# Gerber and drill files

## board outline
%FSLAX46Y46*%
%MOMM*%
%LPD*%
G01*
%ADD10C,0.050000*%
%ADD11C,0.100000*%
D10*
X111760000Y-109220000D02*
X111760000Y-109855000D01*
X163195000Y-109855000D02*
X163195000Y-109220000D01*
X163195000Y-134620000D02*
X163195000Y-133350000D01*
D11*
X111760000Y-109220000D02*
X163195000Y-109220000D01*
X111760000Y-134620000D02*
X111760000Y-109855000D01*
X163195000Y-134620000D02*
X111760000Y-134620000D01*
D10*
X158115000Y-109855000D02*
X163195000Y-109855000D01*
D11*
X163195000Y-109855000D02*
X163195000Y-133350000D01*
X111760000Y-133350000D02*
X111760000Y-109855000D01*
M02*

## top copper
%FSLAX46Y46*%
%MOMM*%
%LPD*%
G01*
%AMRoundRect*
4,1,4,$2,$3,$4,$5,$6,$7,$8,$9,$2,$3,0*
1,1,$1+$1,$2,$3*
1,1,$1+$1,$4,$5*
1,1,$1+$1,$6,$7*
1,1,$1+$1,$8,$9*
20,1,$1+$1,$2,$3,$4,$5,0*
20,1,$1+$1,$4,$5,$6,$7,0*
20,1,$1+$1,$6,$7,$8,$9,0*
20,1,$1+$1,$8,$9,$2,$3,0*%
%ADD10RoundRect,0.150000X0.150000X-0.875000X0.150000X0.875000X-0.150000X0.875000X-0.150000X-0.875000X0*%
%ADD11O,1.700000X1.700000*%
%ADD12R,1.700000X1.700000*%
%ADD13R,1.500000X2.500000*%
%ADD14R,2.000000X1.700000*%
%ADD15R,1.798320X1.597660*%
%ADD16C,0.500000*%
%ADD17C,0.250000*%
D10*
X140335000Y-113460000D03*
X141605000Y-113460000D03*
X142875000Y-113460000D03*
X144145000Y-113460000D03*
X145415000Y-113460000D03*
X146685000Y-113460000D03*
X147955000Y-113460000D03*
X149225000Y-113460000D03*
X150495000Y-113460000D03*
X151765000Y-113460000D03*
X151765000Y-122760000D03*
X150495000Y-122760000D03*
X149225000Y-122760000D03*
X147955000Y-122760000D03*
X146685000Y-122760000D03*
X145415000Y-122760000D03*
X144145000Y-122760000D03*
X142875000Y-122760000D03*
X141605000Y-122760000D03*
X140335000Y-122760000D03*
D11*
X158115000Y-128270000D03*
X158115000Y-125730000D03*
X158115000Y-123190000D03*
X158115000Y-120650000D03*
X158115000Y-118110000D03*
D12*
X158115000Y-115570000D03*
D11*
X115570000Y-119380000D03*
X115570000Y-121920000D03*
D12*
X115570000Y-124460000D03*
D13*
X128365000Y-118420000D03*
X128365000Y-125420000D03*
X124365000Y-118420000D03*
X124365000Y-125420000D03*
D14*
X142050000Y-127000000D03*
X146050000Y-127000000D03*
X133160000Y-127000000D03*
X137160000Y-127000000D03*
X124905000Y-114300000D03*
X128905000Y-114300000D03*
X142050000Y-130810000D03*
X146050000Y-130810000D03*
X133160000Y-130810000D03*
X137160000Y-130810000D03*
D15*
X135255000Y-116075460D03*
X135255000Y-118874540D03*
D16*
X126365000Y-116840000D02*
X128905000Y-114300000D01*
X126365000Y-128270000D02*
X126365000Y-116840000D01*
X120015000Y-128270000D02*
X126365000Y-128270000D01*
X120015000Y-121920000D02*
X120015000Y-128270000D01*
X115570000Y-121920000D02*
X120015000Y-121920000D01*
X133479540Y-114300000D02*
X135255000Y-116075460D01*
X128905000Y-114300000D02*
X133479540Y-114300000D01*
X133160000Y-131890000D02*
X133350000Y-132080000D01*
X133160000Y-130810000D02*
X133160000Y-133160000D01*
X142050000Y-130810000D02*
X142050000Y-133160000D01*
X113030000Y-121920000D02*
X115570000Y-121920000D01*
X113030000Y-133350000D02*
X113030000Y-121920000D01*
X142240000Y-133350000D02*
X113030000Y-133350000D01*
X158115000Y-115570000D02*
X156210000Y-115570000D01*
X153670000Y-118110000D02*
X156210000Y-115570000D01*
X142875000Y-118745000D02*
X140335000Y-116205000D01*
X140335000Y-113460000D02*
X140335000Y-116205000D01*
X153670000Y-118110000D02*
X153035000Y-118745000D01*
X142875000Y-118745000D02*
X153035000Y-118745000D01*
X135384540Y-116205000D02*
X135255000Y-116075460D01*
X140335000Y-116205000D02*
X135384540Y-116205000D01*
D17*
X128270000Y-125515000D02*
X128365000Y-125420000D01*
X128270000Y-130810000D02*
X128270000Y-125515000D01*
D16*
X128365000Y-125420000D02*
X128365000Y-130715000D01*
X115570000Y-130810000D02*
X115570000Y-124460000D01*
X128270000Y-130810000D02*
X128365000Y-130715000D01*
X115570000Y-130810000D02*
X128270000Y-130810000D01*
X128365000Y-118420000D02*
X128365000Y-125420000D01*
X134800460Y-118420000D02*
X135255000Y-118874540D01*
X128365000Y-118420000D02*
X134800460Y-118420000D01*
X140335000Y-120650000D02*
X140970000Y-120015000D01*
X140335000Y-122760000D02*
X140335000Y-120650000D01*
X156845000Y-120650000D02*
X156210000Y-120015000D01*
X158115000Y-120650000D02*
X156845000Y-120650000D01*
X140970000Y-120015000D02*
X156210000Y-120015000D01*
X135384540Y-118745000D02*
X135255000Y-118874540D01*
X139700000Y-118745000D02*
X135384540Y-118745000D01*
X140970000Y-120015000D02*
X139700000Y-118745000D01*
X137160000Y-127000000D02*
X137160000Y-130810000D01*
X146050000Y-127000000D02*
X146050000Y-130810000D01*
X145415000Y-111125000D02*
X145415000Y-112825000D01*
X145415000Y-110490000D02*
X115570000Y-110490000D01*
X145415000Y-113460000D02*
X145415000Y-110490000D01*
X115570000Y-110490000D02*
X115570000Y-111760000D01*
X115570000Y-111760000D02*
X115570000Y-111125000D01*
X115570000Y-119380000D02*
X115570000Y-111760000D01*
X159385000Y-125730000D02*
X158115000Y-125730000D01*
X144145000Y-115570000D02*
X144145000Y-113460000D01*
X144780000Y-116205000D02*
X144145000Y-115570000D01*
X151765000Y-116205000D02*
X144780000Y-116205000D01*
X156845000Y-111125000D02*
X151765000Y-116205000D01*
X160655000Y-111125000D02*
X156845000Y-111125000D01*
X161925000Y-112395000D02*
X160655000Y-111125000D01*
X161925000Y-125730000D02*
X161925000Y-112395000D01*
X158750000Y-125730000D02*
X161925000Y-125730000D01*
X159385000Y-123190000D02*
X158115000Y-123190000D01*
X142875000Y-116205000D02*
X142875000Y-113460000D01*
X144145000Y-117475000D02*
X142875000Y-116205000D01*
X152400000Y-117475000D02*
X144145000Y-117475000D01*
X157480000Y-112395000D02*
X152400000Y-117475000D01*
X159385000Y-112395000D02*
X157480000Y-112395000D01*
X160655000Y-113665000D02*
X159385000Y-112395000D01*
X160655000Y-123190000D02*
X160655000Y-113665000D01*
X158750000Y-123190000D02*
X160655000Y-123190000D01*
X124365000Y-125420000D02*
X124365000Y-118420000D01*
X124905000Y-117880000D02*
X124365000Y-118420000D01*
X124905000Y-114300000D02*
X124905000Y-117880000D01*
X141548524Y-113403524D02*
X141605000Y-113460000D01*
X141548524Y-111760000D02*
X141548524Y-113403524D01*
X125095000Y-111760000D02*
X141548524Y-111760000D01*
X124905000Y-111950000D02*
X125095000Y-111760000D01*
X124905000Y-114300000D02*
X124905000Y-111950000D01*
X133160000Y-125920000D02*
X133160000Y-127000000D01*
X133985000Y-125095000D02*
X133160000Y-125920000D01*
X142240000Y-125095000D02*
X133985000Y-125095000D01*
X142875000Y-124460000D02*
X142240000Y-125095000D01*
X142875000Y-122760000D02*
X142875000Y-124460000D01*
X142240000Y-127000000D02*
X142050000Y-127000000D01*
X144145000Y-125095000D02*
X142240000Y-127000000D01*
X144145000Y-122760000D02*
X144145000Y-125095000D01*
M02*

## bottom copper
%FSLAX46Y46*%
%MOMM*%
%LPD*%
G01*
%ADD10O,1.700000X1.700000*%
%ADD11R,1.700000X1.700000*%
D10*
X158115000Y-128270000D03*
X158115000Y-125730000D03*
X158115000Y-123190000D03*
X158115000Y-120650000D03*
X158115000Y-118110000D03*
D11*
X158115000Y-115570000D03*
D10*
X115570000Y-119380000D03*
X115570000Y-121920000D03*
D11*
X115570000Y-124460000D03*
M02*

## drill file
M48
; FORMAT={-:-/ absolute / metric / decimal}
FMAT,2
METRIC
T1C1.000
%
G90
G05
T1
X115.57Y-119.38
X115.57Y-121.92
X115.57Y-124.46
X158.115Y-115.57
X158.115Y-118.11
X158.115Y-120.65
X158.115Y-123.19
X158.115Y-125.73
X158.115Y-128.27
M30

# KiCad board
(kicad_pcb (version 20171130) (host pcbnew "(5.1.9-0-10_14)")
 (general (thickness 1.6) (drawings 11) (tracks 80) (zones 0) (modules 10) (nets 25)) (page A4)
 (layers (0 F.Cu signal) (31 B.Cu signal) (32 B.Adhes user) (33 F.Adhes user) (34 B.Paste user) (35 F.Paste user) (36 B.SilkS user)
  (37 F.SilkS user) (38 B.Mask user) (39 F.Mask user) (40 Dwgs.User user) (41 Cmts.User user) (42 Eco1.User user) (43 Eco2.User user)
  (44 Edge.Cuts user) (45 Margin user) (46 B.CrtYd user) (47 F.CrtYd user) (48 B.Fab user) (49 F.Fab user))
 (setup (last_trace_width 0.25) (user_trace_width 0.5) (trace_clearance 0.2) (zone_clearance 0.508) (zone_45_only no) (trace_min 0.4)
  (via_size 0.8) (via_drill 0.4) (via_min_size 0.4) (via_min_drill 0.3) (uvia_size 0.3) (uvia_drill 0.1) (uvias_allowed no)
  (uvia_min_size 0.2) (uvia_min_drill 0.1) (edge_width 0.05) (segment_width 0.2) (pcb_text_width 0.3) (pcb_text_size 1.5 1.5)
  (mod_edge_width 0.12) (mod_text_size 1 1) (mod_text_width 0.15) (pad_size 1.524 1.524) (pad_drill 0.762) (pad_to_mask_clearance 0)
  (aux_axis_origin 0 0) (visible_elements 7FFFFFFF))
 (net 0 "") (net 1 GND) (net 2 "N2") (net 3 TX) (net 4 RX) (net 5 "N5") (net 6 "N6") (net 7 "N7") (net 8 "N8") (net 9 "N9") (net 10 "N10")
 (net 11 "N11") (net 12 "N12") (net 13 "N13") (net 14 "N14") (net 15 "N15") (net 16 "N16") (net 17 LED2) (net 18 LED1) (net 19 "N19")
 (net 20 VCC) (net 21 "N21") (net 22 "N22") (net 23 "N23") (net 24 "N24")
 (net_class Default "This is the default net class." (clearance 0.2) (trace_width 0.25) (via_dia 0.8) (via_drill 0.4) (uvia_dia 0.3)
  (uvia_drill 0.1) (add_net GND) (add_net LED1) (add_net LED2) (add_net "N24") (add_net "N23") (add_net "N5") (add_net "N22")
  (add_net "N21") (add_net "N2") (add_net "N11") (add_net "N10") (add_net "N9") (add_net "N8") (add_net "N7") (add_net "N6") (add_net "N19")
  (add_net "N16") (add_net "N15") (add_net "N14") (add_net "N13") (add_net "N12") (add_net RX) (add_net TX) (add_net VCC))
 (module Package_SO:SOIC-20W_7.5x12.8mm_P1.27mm (layer F.Cu) (at 146.05 118.11 90)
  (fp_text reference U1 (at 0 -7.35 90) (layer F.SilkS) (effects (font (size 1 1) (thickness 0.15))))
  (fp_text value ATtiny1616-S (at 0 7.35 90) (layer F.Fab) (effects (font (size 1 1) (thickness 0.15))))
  (pad 20 smd roundrect (at 4.65 -5.715 90) (size 2.05 0.6) (layers F.Cu F.Paste F.Mask) (roundrect_rratio 0.25) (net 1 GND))
  (pad 19 smd roundrect (at 4.65 -4.445 90) (size 2.05 0.6) (layers F.Cu F.Paste F.Mask) (roundrect_rratio 0.25) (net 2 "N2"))
  (pad 18 smd roundrect (at 4.65 -3.175 90) (size 2.05 0.6) (layers F.Cu F.Paste F.Mask) (roundrect_rratio 0.25) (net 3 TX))
  (pad 17 smd roundrect (at 4.65 -1.905 90) (size 2.05 0.6) (layers F.Cu F.Paste F.Mask) (roundrect_rratio 0.25) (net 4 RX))
  (pad 16 smd roundrect (at 4.65 -0.635 90) (size 2.05 0.6) (layers F.Cu F.Paste F.Mask) (roundrect_rratio 0.25) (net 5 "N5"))
  (pad 15 smd roundrect (at 4.65 0.635 90) (size 2.05 0.6) (layers F.Cu F.Paste F.Mask) (roundrect_rratio 0.25) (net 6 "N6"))
  (pad 14 smd roundrect (at 4.65 1.905 90) (size 2.05 0.6) (layers F.Cu F.Paste F.Mask) (roundrect_rratio 0.25) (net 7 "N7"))
  (pad 13 smd roundrect (at 4.65 3.175 90) (size 2.05 0.6) (layers F.Cu F.Paste F.Mask) (roundrect_rratio 0.25) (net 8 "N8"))
  (pad 12 smd roundrect (at 4.65 4.445 90) (size 2.05 0.6) (layers F.Cu F.Paste F.Mask) (roundrect_rratio 0.25) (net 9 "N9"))
  (pad 11 smd roundrect (at 4.65 5.715 90) (size 2.05 0.6) (layers F.Cu F.Paste F.Mask) (roundrect_rratio 0.25) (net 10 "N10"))
  (pad 10 smd roundrect (at -4.65 5.715 90) (size 2.05 0.6) (layers F.Cu F.Paste F.Mask) (roundrect_rratio 0.25) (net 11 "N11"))
  (pad 9 smd roundrect (at -4.65 4.445 90) (size 2.05 0.6) (layers F.Cu F.Paste F.Mask) (roundrect_rratio 0.25) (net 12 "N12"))
  (pad 8 smd roundrect (at -4.65 3.175 90) (size 2.05 0.6) (layers F.Cu F.Paste F.Mask) (roundrect_rratio 0.25) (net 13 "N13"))
  (pad 7 smd roundrect (at -4.65 1.905 90) (size 2.05 0.6) (layers F.Cu F.Paste F.Mask) (roundrect_rratio 0.25) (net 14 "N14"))
  (pad 6 smd roundrect (at -4.65 0.635 90) (size 2.05 0.6) (layers F.Cu F.Paste F.Mask) (roundrect_rratio 0.25) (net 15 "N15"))
  (pad 5 smd roundrect (at -4.65 -0.635 90) (size 2.05 0.6) (layers F.Cu F.Paste F.Mask) (roundrect_rratio 0.25) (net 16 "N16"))
  (pad 4 smd roundrect (at -4.65 -1.905 90) (size 2.05 0.6) (layers F.Cu F.Paste F.Mask) (roundrect_rratio 0.25) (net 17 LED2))
  (pad 3 smd roundrect (at -4.65 -3.175 90) (size 2.05 0.6) (layers F.Cu F.Paste F.Mask) (roundrect_rratio 0.25) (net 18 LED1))
  (pad 2 smd roundrect (at -4.65 -4.445 90) (size 2.05 0.6) (layers F.Cu F.Paste F.Mask) (roundrect_rratio 0.25) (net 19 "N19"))
  (pad 1 smd roundrect (at -4.65 -5.715 90) (size 2.05 0.6) (layers F.Cu F.Paste F.Mask) (roundrect_rratio 0.25) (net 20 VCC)))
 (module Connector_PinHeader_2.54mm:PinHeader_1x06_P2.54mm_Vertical (layer F.Cu) (at 158.115 115.57)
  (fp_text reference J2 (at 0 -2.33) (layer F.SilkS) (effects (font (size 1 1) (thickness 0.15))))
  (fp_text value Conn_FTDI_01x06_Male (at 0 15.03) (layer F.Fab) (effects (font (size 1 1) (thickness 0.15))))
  (pad 6 thru_hole oval (at 0 12.7) (size 1.7 1.7) (drill 1) (layers *.Cu *.Mask) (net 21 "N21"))
  (pad 5 thru_hole oval (at 0 10.16) (size 1.7 1.7) (drill 1) (layers *.Cu *.Mask) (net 4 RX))
  (pad 4 thru_hole oval (at 0 7.62) (size 1.7 1.7) (drill 1) (layers *.Cu *.Mask) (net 3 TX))
  (pad 3 thru_hole oval (at 0 5.08) (size 1.7 1.7) (drill 1) (layers *.Cu *.Mask) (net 20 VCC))
  (pad 2 thru_hole oval (at 0 2.54) (size 1.7 1.7) (drill 1) (layers *.Cu *.Mask) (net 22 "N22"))
  (pad 1 thru_hole rect (at 0 0) (size 1.7 1.7) (drill 1) (layers *.Cu *.Mask) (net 1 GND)))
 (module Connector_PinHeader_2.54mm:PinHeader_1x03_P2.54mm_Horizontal (layer F.Cu) (at 115.57 124.46 180)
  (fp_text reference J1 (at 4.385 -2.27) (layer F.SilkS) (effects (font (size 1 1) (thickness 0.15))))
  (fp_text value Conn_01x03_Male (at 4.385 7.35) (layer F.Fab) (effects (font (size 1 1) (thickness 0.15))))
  (pad 3 thru_hole oval (at 0 5.08 180) (size 1.7 1.7) (drill 1) (layers *.Cu *.Mask) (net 5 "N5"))
  (pad 2 thru_hole oval (at 0 2.54 180) (size 1.7 1.7) (drill 1) (layers *.Cu *.Mask) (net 1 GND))
  (pad 1 thru_hole rect (at 0 0 180) (size 1.7 1.7) (drill 1) (layers *.Cu *.Mask) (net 20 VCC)))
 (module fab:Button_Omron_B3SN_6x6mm (layer F.Cu) (at 126.365 121.92 270)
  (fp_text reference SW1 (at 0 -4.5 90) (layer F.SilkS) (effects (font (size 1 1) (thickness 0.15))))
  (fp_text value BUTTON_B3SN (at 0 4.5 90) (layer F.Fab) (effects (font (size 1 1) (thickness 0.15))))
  (pad 1 smd rect (at -3.5 -2 270) (size 2.5 1.5) (layers F.Cu F.Paste F.Mask) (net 20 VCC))
  (pad 1 smd rect (at 3.5 -2 270) (size 2.5 1.5) (layers F.Cu F.Paste F.Mask) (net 20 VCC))
  (pad 2 smd rect (at -3.5 2 270) (size 2.5 1.5) (layers F.Cu F.Paste F.Mask) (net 2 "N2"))
  (pad 2 smd rect (at 3.5 2 270) (size 2.5 1.5) (layers F.Cu F.Paste F.Mask) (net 2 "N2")))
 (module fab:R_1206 (layer F.Cu) (at 144.05 127)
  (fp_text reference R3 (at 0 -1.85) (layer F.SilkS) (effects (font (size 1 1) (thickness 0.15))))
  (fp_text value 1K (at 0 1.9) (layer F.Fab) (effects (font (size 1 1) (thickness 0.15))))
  (pad 1 smd rect (at -2 0) (size 2 1.7) (layers F.Cu F.Paste F.Mask) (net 17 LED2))
  (pad 2 smd rect (at 2 0) (size 2 1.7) (layers F.Cu F.Paste F.Mask) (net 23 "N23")))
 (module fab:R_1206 (layer F.Cu) (at 135.16 127)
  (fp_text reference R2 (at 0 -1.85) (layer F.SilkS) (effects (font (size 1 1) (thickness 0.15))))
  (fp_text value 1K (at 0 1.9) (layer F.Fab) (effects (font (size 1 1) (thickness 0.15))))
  (pad 1 smd rect (at -2 0) (size 2 1.7) (layers F.Cu F.Paste F.Mask) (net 18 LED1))
  (pad 2 smd rect (at 2 0) (size 2 1.7) (layers F.Cu F.Paste F.Mask) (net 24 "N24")))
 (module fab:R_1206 (layer F.Cu) (at 126.905 114.3)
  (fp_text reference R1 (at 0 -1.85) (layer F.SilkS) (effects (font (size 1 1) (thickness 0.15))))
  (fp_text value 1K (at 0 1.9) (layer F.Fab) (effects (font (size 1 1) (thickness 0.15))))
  (pad 1 smd rect (at -2 0) (size 2 1.7) (layers F.Cu F.Paste F.Mask) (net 2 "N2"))
  (pad 2 smd rect (at 2 0) (size 2 1.7) (layers F.Cu F.Paste F.Mask) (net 1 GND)))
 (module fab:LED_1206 (layer F.Cu) (at 144.05 130.81)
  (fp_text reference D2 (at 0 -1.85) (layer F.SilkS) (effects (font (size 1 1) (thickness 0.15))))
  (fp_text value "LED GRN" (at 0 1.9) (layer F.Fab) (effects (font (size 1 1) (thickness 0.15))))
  (pad 1 smd rect (at -2 0) (size 2 1.7) (layers F.Cu F.Paste F.Mask) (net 1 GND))
  (pad 2 smd rect (at 2 0) (size 2 1.7) (layers F.Cu F.Paste F.Mask) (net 23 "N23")))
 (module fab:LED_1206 (layer F.Cu) (at 135.16 130.81)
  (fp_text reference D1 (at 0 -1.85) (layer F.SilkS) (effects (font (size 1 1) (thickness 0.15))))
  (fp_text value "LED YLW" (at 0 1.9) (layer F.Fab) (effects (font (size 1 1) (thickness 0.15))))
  (pad 1 smd rect (at -2 0) (size 2 1.7) (layers F.Cu F.Paste F.Mask) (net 1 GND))
  (pad 2 smd rect (at 2 0) (size 2 1.7) (layers F.Cu F.Paste F.Mask) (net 24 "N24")))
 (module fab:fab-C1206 (layer F.Cu) (at 135.255 117.475 90)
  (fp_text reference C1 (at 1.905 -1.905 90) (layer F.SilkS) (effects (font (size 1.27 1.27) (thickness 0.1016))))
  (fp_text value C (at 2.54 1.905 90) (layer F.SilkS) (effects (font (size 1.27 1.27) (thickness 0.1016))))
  (pad 2 smd rect (at 1.39954 0 90) (size 1.59766 1.79832) (layers F.Cu F.Paste F.Mask) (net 1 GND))
  (pad 1 smd rect (at -1.39954 0 90) (size 1.59766 1.79832) (layers F.Cu F.Paste F.Mask) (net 20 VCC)))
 (gr_line (start 111.76 109.22) (end 111.76 109.855) (layer Edge.Cuts) (width 0.05))
 (gr_line (start 163.195 109.855) (end 163.195 109.22) (layer Edge.Cuts) (width 0.05))
 (gr_line (start 163.195 134.62) (end 163.195 133.35) (layer Edge.Cuts) (width 0.05))
 (gr_line (start 111.76 109.22) (end 163.195 109.22) (layer Edge.Cuts) (width 0.1))
 (gr_line (start 111.76 134.62) (end 111.76 109.855) (layer Edge.Cuts) (width 0.1))
 (gr_line (start 163.195 134.62) (end 111.76 134.62) (layer Edge.Cuts) (width 0.1))
 (gr_line (start 158.115 109.855) (end 163.195 109.855) (layer Edge.Cuts) (width 0.05))
 (gr_line (start 163.195 109.855) (end 163.195 133.35) (layer Edge.Cuts) (width 0.1))
 (gr_line (start 111.76 133.35) (end 111.76 109.855) (layer Edge.Cuts) (width 0.1))
 (segment (start 126.365 116.84) (end 128.905 114.3) (width 0.5) (layer F.Cu) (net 1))
 (segment (start 126.365 128.27) (end 126.365 116.84) (width 0.5) (layer F.Cu) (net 1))
 (segment (start 120.015 128.27) (end 126.365 128.27) (width 0.5) (layer F.Cu) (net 1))
 (segment (start 120.015 121.92) (end 120.015 128.27) (width 0.5) (layer F.Cu) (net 1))
 (segment (start 115.57 121.92) (end 120.015 121.92) (width 0.5) (layer F.Cu) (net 1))
 (segment (start 133.47954 114.3) (end 135.255 116.07546) (width 0.5) (layer F.Cu) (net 1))
 (segment (start 128.905 114.3) (end 133.47954 114.3) (width 0.5) (layer F.Cu) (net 1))
 (segment (start 133.16 131.89) (end 133.35 132.08) (width 0.5) (layer F.Cu) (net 1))
 (segment (start 133.16 130.81) (end 133.16 133.16) (width 0.5) (layer F.Cu) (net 1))
 (segment (start 142.05 130.81) (end 142.05 133.16) (width 0.5) (layer F.Cu) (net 1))
 (segment (start 113.03 121.92) (end 115.57 121.92) (width 0.5) (layer F.Cu) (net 1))
 (segment (start 113.03 133.35) (end 113.03 121.92) (width 0.5) (layer F.Cu) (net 1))
 (segment (start 142.24 133.35) (end 113.03 133.35) (width 0.5) (layer F.Cu) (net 1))
 (segment (start 158.115 115.57) (end 156.21 115.57) (width 0.5) (layer F.Cu) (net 1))
 (segment (start 153.67 118.11) (end 156.21 115.57) (width 0.5) (layer F.Cu) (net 1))
 (segment (start 142.875 118.745) (end 140.335 116.205) (width 0.5) (layer F.Cu) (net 1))
 (segment (start 140.335 113.46) (end 140.335 116.205) (width 0.5) (layer F.Cu) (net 1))
 (segment (start 153.67 118.11) (end 153.035 118.745) (width 0.5) (layer F.Cu) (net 1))
 (segment (start 142.875 118.745) (end 153.035 118.745) (width 0.5) (layer F.Cu) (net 1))
 (segment (start 135.38454 116.205) (end 135.255 116.07546) (width 0.5) (layer F.Cu) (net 1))
 (segment (start 140.335 116.205) (end 135.38454 116.205) (width 0.5) (layer F.Cu) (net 1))
 (segment (start 128.27 125.515) (end 128.365 125.42) (width 0.25) (layer F.Cu) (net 20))
 (segment (start 128.27 130.81) (end 128.27 125.515) (width 0.25) (layer F.Cu) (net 20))
 (segment (start 128.365 125.42) (end 128.365 130.715) (width 0.5) (layer F.Cu) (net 20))
 (segment (start 115.57 130.81) (end 115.57 124.46) (width 0.5) (layer F.Cu) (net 20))
 (segment (start 128.27 130.81) (end 128.365 130.715) (width 0.5) (layer F.Cu) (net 20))
 (segment (start 115.57 130.81) (end 128.27 130.81) (width 0.5) (layer F.Cu) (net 20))
 (segment (start 128.365 118.42) (end 128.365 125.42) (width 0.5) (layer F.Cu) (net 20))
 (segment (start 134.80046 118.42) (end 135.255 118.87454) (width 0.5) (layer F.Cu) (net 20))
 (segment (start 128.365 118.42) (end 134.80046 118.42) (width 0.5) (layer F.Cu) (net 20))
 (segment (start 140.335 120.65) (end 140.97 120.015) (width 0.5) (layer F.Cu) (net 20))
 (segment (start 140.335 122.76) (end 140.335 120.65) (width 0.5) (layer F.Cu) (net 20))
 (segment (start 156.845 120.65) (end 156.21 120.015) (width 0.5) (layer F.Cu) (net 20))
 (segment (start 158.115 120.65) (end 156.845 120.65) (width 0.5) (layer F.Cu) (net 20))
 (segment (start 140.97 120.015) (end 156.21 120.015) (width 0.5) (layer F.Cu) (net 20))
 (segment (start 135.38454 118.745) (end 135.255 118.87454) (width 0.5) (layer F.Cu) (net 20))
 (segment (start 139.7 118.745) (end 135.38454 118.745) (width 0.5) (layer F.Cu) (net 20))
 (segment (start 140.97 120.015) (end 139.7 118.745) (width 0.5) (layer F.Cu) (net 20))
 (segment (start 137.16 127) (end 137.16 130.81) (width 0.5) (layer F.Cu) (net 24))
 (segment (start 146.05 127) (end 146.05 130.81) (width 0.5) (layer F.Cu) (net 23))
 (segment (start 145.415 111.125) (end 145.415 112.825) (width 0.5) (layer F.Cu) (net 5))
 (segment (start 145.415 110.49) (end 115.57 110.49) (width 0.5) (layer F.Cu) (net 5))
 (segment (start 145.415 113.46) (end 145.415 110.49) (width 0.5) (layer F.Cu) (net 5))
 (segment (start 115.57 110.49) (end 115.57 111.76) (width 0.5) (layer F.Cu) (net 5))
 (segment (start 115.57 111.76) (end 115.57 111.125) (width 0.5) (layer F.Cu) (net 5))
 (segment (start 115.57 119.38) (end 115.57 111.76) (width 0.5) (layer F.Cu) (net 5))
 (segment (start 159.385 125.73) (end 158.115 125.73) (width 0.5) (layer F.Cu) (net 4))
 (segment (start 144.145 115.57) (end 144.145 113.46) (width 0.5) (layer F.Cu) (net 4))
 (segment (start 144.78 116.205) (end 144.145 115.57) (width 0.5) (layer F.Cu) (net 4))
 (segment (start 151.765 116.205) (end 144.78 116.205) (width 0.5) (layer F.Cu) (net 4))
 (segment (start 156.845 111.125) (end 151.765 116.205) (width 0.5) (layer F.Cu) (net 4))
 (segment (start 160.655 111.125) (end 156.845 111.125) (width 0.5) (layer F.Cu) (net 4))
 (segment (start 161.925 112.395) (end 160.655 111.125) (width 0.5) (layer F.Cu) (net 4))
 (segment (start 161.925 125.73) (end 161.925 112.395) (width 0.5) (layer F.Cu) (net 4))
 (segment (start 158.75 125.73) (end 161.925 125.73) (width 0.5) (layer F.Cu) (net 4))
 (segment (start 159.385 123.19) (end 158.115 123.19) (width 0.5) (layer F.Cu) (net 3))
 (segment (start 142.875 116.205) (end 142.875 113.46) (width 0.5) (layer F.Cu) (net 3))
 (segment (start 144.145 117.475) (end 142.875 116.205) (width 0.5) (layer F.Cu) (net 3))
 (segment (start 152.4 117.475) (end 144.145 117.475) (width 0.5) (layer F.Cu) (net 3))
 (segment (start 157.48 112.395) (end 152.4 117.475) (width 0.5) (layer F.Cu) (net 3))
 (segment (start 159.385 112.395) (end 157.48 112.395) (width 0.5) (layer F.Cu) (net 3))
 (segment (start 160.655 113.665) (end 159.385 112.395) (width 0.5) (layer F.Cu) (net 3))
 (segment (start 160.655 123.19) (end 160.655 113.665) (width 0.5) (layer F.Cu) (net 3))
 (segment (start 158.75 123.19) (end 160.655 123.19) (width 0.5) (layer F.Cu) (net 3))
 (segment (start 124.365 125.42) (end 124.365 118.42) (width 0.5) (layer F.Cu) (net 2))
 (segment (start 124.905 117.88) (end 124.365 118.42) (width 0.5) (layer F.Cu) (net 2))
 (segment (start 124.905 114.3) (end 124.905 117.88) (width 0.5) (layer F.Cu) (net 2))
 (segment (start 141.548524 113.403524) (end 141.605 113.46) (width 0.5) (layer F.Cu) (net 2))
 (segment (start 141.548524 111.76) (end 141.548524 113.403524) (width 0.5) (layer F.Cu) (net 2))
 (segment (start 125.095 111.76) (end 141.548524 111.76) (width 0.5) (layer F.Cu) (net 2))
 (segment (start 124.905 111.95) (end 125.095 111.76) (width 0.5) (layer F.Cu) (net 2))
 (segment (start 124.905 114.3) (end 124.905 111.95) (width 0.5) (layer F.Cu) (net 2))
 (segment (start 133.16 125.92) (end 133.16 127) (width 0.5) (layer F.Cu) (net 18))
 (segment (start 133.985 125.095) (end 133.16 125.92) (width 0.5) (layer F.Cu) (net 18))
 (segment (start 142.24 125.095) (end 133.985 125.095) (width 0.5) (layer F.Cu) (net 18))
 (segment (start 142.875 124.46) (end 142.24 125.095) (width 0.5) (layer F.Cu) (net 18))
 (segment (start 142.875 122.76) (end 142.875 124.46) (width 0.5) (layer F.Cu) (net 18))
 (segment (start 142.24 127) (end 142.05 127) (width 0.5) (layer F.Cu) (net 17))
 (segment (start 144.145 125.095) (end 142.24 127) (width 0.5) (layer F.Cu) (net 17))
 (segment (start 144.145 122.76) (end 144.145 125.095) (width 0.5) (layer F.Cu) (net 17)))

